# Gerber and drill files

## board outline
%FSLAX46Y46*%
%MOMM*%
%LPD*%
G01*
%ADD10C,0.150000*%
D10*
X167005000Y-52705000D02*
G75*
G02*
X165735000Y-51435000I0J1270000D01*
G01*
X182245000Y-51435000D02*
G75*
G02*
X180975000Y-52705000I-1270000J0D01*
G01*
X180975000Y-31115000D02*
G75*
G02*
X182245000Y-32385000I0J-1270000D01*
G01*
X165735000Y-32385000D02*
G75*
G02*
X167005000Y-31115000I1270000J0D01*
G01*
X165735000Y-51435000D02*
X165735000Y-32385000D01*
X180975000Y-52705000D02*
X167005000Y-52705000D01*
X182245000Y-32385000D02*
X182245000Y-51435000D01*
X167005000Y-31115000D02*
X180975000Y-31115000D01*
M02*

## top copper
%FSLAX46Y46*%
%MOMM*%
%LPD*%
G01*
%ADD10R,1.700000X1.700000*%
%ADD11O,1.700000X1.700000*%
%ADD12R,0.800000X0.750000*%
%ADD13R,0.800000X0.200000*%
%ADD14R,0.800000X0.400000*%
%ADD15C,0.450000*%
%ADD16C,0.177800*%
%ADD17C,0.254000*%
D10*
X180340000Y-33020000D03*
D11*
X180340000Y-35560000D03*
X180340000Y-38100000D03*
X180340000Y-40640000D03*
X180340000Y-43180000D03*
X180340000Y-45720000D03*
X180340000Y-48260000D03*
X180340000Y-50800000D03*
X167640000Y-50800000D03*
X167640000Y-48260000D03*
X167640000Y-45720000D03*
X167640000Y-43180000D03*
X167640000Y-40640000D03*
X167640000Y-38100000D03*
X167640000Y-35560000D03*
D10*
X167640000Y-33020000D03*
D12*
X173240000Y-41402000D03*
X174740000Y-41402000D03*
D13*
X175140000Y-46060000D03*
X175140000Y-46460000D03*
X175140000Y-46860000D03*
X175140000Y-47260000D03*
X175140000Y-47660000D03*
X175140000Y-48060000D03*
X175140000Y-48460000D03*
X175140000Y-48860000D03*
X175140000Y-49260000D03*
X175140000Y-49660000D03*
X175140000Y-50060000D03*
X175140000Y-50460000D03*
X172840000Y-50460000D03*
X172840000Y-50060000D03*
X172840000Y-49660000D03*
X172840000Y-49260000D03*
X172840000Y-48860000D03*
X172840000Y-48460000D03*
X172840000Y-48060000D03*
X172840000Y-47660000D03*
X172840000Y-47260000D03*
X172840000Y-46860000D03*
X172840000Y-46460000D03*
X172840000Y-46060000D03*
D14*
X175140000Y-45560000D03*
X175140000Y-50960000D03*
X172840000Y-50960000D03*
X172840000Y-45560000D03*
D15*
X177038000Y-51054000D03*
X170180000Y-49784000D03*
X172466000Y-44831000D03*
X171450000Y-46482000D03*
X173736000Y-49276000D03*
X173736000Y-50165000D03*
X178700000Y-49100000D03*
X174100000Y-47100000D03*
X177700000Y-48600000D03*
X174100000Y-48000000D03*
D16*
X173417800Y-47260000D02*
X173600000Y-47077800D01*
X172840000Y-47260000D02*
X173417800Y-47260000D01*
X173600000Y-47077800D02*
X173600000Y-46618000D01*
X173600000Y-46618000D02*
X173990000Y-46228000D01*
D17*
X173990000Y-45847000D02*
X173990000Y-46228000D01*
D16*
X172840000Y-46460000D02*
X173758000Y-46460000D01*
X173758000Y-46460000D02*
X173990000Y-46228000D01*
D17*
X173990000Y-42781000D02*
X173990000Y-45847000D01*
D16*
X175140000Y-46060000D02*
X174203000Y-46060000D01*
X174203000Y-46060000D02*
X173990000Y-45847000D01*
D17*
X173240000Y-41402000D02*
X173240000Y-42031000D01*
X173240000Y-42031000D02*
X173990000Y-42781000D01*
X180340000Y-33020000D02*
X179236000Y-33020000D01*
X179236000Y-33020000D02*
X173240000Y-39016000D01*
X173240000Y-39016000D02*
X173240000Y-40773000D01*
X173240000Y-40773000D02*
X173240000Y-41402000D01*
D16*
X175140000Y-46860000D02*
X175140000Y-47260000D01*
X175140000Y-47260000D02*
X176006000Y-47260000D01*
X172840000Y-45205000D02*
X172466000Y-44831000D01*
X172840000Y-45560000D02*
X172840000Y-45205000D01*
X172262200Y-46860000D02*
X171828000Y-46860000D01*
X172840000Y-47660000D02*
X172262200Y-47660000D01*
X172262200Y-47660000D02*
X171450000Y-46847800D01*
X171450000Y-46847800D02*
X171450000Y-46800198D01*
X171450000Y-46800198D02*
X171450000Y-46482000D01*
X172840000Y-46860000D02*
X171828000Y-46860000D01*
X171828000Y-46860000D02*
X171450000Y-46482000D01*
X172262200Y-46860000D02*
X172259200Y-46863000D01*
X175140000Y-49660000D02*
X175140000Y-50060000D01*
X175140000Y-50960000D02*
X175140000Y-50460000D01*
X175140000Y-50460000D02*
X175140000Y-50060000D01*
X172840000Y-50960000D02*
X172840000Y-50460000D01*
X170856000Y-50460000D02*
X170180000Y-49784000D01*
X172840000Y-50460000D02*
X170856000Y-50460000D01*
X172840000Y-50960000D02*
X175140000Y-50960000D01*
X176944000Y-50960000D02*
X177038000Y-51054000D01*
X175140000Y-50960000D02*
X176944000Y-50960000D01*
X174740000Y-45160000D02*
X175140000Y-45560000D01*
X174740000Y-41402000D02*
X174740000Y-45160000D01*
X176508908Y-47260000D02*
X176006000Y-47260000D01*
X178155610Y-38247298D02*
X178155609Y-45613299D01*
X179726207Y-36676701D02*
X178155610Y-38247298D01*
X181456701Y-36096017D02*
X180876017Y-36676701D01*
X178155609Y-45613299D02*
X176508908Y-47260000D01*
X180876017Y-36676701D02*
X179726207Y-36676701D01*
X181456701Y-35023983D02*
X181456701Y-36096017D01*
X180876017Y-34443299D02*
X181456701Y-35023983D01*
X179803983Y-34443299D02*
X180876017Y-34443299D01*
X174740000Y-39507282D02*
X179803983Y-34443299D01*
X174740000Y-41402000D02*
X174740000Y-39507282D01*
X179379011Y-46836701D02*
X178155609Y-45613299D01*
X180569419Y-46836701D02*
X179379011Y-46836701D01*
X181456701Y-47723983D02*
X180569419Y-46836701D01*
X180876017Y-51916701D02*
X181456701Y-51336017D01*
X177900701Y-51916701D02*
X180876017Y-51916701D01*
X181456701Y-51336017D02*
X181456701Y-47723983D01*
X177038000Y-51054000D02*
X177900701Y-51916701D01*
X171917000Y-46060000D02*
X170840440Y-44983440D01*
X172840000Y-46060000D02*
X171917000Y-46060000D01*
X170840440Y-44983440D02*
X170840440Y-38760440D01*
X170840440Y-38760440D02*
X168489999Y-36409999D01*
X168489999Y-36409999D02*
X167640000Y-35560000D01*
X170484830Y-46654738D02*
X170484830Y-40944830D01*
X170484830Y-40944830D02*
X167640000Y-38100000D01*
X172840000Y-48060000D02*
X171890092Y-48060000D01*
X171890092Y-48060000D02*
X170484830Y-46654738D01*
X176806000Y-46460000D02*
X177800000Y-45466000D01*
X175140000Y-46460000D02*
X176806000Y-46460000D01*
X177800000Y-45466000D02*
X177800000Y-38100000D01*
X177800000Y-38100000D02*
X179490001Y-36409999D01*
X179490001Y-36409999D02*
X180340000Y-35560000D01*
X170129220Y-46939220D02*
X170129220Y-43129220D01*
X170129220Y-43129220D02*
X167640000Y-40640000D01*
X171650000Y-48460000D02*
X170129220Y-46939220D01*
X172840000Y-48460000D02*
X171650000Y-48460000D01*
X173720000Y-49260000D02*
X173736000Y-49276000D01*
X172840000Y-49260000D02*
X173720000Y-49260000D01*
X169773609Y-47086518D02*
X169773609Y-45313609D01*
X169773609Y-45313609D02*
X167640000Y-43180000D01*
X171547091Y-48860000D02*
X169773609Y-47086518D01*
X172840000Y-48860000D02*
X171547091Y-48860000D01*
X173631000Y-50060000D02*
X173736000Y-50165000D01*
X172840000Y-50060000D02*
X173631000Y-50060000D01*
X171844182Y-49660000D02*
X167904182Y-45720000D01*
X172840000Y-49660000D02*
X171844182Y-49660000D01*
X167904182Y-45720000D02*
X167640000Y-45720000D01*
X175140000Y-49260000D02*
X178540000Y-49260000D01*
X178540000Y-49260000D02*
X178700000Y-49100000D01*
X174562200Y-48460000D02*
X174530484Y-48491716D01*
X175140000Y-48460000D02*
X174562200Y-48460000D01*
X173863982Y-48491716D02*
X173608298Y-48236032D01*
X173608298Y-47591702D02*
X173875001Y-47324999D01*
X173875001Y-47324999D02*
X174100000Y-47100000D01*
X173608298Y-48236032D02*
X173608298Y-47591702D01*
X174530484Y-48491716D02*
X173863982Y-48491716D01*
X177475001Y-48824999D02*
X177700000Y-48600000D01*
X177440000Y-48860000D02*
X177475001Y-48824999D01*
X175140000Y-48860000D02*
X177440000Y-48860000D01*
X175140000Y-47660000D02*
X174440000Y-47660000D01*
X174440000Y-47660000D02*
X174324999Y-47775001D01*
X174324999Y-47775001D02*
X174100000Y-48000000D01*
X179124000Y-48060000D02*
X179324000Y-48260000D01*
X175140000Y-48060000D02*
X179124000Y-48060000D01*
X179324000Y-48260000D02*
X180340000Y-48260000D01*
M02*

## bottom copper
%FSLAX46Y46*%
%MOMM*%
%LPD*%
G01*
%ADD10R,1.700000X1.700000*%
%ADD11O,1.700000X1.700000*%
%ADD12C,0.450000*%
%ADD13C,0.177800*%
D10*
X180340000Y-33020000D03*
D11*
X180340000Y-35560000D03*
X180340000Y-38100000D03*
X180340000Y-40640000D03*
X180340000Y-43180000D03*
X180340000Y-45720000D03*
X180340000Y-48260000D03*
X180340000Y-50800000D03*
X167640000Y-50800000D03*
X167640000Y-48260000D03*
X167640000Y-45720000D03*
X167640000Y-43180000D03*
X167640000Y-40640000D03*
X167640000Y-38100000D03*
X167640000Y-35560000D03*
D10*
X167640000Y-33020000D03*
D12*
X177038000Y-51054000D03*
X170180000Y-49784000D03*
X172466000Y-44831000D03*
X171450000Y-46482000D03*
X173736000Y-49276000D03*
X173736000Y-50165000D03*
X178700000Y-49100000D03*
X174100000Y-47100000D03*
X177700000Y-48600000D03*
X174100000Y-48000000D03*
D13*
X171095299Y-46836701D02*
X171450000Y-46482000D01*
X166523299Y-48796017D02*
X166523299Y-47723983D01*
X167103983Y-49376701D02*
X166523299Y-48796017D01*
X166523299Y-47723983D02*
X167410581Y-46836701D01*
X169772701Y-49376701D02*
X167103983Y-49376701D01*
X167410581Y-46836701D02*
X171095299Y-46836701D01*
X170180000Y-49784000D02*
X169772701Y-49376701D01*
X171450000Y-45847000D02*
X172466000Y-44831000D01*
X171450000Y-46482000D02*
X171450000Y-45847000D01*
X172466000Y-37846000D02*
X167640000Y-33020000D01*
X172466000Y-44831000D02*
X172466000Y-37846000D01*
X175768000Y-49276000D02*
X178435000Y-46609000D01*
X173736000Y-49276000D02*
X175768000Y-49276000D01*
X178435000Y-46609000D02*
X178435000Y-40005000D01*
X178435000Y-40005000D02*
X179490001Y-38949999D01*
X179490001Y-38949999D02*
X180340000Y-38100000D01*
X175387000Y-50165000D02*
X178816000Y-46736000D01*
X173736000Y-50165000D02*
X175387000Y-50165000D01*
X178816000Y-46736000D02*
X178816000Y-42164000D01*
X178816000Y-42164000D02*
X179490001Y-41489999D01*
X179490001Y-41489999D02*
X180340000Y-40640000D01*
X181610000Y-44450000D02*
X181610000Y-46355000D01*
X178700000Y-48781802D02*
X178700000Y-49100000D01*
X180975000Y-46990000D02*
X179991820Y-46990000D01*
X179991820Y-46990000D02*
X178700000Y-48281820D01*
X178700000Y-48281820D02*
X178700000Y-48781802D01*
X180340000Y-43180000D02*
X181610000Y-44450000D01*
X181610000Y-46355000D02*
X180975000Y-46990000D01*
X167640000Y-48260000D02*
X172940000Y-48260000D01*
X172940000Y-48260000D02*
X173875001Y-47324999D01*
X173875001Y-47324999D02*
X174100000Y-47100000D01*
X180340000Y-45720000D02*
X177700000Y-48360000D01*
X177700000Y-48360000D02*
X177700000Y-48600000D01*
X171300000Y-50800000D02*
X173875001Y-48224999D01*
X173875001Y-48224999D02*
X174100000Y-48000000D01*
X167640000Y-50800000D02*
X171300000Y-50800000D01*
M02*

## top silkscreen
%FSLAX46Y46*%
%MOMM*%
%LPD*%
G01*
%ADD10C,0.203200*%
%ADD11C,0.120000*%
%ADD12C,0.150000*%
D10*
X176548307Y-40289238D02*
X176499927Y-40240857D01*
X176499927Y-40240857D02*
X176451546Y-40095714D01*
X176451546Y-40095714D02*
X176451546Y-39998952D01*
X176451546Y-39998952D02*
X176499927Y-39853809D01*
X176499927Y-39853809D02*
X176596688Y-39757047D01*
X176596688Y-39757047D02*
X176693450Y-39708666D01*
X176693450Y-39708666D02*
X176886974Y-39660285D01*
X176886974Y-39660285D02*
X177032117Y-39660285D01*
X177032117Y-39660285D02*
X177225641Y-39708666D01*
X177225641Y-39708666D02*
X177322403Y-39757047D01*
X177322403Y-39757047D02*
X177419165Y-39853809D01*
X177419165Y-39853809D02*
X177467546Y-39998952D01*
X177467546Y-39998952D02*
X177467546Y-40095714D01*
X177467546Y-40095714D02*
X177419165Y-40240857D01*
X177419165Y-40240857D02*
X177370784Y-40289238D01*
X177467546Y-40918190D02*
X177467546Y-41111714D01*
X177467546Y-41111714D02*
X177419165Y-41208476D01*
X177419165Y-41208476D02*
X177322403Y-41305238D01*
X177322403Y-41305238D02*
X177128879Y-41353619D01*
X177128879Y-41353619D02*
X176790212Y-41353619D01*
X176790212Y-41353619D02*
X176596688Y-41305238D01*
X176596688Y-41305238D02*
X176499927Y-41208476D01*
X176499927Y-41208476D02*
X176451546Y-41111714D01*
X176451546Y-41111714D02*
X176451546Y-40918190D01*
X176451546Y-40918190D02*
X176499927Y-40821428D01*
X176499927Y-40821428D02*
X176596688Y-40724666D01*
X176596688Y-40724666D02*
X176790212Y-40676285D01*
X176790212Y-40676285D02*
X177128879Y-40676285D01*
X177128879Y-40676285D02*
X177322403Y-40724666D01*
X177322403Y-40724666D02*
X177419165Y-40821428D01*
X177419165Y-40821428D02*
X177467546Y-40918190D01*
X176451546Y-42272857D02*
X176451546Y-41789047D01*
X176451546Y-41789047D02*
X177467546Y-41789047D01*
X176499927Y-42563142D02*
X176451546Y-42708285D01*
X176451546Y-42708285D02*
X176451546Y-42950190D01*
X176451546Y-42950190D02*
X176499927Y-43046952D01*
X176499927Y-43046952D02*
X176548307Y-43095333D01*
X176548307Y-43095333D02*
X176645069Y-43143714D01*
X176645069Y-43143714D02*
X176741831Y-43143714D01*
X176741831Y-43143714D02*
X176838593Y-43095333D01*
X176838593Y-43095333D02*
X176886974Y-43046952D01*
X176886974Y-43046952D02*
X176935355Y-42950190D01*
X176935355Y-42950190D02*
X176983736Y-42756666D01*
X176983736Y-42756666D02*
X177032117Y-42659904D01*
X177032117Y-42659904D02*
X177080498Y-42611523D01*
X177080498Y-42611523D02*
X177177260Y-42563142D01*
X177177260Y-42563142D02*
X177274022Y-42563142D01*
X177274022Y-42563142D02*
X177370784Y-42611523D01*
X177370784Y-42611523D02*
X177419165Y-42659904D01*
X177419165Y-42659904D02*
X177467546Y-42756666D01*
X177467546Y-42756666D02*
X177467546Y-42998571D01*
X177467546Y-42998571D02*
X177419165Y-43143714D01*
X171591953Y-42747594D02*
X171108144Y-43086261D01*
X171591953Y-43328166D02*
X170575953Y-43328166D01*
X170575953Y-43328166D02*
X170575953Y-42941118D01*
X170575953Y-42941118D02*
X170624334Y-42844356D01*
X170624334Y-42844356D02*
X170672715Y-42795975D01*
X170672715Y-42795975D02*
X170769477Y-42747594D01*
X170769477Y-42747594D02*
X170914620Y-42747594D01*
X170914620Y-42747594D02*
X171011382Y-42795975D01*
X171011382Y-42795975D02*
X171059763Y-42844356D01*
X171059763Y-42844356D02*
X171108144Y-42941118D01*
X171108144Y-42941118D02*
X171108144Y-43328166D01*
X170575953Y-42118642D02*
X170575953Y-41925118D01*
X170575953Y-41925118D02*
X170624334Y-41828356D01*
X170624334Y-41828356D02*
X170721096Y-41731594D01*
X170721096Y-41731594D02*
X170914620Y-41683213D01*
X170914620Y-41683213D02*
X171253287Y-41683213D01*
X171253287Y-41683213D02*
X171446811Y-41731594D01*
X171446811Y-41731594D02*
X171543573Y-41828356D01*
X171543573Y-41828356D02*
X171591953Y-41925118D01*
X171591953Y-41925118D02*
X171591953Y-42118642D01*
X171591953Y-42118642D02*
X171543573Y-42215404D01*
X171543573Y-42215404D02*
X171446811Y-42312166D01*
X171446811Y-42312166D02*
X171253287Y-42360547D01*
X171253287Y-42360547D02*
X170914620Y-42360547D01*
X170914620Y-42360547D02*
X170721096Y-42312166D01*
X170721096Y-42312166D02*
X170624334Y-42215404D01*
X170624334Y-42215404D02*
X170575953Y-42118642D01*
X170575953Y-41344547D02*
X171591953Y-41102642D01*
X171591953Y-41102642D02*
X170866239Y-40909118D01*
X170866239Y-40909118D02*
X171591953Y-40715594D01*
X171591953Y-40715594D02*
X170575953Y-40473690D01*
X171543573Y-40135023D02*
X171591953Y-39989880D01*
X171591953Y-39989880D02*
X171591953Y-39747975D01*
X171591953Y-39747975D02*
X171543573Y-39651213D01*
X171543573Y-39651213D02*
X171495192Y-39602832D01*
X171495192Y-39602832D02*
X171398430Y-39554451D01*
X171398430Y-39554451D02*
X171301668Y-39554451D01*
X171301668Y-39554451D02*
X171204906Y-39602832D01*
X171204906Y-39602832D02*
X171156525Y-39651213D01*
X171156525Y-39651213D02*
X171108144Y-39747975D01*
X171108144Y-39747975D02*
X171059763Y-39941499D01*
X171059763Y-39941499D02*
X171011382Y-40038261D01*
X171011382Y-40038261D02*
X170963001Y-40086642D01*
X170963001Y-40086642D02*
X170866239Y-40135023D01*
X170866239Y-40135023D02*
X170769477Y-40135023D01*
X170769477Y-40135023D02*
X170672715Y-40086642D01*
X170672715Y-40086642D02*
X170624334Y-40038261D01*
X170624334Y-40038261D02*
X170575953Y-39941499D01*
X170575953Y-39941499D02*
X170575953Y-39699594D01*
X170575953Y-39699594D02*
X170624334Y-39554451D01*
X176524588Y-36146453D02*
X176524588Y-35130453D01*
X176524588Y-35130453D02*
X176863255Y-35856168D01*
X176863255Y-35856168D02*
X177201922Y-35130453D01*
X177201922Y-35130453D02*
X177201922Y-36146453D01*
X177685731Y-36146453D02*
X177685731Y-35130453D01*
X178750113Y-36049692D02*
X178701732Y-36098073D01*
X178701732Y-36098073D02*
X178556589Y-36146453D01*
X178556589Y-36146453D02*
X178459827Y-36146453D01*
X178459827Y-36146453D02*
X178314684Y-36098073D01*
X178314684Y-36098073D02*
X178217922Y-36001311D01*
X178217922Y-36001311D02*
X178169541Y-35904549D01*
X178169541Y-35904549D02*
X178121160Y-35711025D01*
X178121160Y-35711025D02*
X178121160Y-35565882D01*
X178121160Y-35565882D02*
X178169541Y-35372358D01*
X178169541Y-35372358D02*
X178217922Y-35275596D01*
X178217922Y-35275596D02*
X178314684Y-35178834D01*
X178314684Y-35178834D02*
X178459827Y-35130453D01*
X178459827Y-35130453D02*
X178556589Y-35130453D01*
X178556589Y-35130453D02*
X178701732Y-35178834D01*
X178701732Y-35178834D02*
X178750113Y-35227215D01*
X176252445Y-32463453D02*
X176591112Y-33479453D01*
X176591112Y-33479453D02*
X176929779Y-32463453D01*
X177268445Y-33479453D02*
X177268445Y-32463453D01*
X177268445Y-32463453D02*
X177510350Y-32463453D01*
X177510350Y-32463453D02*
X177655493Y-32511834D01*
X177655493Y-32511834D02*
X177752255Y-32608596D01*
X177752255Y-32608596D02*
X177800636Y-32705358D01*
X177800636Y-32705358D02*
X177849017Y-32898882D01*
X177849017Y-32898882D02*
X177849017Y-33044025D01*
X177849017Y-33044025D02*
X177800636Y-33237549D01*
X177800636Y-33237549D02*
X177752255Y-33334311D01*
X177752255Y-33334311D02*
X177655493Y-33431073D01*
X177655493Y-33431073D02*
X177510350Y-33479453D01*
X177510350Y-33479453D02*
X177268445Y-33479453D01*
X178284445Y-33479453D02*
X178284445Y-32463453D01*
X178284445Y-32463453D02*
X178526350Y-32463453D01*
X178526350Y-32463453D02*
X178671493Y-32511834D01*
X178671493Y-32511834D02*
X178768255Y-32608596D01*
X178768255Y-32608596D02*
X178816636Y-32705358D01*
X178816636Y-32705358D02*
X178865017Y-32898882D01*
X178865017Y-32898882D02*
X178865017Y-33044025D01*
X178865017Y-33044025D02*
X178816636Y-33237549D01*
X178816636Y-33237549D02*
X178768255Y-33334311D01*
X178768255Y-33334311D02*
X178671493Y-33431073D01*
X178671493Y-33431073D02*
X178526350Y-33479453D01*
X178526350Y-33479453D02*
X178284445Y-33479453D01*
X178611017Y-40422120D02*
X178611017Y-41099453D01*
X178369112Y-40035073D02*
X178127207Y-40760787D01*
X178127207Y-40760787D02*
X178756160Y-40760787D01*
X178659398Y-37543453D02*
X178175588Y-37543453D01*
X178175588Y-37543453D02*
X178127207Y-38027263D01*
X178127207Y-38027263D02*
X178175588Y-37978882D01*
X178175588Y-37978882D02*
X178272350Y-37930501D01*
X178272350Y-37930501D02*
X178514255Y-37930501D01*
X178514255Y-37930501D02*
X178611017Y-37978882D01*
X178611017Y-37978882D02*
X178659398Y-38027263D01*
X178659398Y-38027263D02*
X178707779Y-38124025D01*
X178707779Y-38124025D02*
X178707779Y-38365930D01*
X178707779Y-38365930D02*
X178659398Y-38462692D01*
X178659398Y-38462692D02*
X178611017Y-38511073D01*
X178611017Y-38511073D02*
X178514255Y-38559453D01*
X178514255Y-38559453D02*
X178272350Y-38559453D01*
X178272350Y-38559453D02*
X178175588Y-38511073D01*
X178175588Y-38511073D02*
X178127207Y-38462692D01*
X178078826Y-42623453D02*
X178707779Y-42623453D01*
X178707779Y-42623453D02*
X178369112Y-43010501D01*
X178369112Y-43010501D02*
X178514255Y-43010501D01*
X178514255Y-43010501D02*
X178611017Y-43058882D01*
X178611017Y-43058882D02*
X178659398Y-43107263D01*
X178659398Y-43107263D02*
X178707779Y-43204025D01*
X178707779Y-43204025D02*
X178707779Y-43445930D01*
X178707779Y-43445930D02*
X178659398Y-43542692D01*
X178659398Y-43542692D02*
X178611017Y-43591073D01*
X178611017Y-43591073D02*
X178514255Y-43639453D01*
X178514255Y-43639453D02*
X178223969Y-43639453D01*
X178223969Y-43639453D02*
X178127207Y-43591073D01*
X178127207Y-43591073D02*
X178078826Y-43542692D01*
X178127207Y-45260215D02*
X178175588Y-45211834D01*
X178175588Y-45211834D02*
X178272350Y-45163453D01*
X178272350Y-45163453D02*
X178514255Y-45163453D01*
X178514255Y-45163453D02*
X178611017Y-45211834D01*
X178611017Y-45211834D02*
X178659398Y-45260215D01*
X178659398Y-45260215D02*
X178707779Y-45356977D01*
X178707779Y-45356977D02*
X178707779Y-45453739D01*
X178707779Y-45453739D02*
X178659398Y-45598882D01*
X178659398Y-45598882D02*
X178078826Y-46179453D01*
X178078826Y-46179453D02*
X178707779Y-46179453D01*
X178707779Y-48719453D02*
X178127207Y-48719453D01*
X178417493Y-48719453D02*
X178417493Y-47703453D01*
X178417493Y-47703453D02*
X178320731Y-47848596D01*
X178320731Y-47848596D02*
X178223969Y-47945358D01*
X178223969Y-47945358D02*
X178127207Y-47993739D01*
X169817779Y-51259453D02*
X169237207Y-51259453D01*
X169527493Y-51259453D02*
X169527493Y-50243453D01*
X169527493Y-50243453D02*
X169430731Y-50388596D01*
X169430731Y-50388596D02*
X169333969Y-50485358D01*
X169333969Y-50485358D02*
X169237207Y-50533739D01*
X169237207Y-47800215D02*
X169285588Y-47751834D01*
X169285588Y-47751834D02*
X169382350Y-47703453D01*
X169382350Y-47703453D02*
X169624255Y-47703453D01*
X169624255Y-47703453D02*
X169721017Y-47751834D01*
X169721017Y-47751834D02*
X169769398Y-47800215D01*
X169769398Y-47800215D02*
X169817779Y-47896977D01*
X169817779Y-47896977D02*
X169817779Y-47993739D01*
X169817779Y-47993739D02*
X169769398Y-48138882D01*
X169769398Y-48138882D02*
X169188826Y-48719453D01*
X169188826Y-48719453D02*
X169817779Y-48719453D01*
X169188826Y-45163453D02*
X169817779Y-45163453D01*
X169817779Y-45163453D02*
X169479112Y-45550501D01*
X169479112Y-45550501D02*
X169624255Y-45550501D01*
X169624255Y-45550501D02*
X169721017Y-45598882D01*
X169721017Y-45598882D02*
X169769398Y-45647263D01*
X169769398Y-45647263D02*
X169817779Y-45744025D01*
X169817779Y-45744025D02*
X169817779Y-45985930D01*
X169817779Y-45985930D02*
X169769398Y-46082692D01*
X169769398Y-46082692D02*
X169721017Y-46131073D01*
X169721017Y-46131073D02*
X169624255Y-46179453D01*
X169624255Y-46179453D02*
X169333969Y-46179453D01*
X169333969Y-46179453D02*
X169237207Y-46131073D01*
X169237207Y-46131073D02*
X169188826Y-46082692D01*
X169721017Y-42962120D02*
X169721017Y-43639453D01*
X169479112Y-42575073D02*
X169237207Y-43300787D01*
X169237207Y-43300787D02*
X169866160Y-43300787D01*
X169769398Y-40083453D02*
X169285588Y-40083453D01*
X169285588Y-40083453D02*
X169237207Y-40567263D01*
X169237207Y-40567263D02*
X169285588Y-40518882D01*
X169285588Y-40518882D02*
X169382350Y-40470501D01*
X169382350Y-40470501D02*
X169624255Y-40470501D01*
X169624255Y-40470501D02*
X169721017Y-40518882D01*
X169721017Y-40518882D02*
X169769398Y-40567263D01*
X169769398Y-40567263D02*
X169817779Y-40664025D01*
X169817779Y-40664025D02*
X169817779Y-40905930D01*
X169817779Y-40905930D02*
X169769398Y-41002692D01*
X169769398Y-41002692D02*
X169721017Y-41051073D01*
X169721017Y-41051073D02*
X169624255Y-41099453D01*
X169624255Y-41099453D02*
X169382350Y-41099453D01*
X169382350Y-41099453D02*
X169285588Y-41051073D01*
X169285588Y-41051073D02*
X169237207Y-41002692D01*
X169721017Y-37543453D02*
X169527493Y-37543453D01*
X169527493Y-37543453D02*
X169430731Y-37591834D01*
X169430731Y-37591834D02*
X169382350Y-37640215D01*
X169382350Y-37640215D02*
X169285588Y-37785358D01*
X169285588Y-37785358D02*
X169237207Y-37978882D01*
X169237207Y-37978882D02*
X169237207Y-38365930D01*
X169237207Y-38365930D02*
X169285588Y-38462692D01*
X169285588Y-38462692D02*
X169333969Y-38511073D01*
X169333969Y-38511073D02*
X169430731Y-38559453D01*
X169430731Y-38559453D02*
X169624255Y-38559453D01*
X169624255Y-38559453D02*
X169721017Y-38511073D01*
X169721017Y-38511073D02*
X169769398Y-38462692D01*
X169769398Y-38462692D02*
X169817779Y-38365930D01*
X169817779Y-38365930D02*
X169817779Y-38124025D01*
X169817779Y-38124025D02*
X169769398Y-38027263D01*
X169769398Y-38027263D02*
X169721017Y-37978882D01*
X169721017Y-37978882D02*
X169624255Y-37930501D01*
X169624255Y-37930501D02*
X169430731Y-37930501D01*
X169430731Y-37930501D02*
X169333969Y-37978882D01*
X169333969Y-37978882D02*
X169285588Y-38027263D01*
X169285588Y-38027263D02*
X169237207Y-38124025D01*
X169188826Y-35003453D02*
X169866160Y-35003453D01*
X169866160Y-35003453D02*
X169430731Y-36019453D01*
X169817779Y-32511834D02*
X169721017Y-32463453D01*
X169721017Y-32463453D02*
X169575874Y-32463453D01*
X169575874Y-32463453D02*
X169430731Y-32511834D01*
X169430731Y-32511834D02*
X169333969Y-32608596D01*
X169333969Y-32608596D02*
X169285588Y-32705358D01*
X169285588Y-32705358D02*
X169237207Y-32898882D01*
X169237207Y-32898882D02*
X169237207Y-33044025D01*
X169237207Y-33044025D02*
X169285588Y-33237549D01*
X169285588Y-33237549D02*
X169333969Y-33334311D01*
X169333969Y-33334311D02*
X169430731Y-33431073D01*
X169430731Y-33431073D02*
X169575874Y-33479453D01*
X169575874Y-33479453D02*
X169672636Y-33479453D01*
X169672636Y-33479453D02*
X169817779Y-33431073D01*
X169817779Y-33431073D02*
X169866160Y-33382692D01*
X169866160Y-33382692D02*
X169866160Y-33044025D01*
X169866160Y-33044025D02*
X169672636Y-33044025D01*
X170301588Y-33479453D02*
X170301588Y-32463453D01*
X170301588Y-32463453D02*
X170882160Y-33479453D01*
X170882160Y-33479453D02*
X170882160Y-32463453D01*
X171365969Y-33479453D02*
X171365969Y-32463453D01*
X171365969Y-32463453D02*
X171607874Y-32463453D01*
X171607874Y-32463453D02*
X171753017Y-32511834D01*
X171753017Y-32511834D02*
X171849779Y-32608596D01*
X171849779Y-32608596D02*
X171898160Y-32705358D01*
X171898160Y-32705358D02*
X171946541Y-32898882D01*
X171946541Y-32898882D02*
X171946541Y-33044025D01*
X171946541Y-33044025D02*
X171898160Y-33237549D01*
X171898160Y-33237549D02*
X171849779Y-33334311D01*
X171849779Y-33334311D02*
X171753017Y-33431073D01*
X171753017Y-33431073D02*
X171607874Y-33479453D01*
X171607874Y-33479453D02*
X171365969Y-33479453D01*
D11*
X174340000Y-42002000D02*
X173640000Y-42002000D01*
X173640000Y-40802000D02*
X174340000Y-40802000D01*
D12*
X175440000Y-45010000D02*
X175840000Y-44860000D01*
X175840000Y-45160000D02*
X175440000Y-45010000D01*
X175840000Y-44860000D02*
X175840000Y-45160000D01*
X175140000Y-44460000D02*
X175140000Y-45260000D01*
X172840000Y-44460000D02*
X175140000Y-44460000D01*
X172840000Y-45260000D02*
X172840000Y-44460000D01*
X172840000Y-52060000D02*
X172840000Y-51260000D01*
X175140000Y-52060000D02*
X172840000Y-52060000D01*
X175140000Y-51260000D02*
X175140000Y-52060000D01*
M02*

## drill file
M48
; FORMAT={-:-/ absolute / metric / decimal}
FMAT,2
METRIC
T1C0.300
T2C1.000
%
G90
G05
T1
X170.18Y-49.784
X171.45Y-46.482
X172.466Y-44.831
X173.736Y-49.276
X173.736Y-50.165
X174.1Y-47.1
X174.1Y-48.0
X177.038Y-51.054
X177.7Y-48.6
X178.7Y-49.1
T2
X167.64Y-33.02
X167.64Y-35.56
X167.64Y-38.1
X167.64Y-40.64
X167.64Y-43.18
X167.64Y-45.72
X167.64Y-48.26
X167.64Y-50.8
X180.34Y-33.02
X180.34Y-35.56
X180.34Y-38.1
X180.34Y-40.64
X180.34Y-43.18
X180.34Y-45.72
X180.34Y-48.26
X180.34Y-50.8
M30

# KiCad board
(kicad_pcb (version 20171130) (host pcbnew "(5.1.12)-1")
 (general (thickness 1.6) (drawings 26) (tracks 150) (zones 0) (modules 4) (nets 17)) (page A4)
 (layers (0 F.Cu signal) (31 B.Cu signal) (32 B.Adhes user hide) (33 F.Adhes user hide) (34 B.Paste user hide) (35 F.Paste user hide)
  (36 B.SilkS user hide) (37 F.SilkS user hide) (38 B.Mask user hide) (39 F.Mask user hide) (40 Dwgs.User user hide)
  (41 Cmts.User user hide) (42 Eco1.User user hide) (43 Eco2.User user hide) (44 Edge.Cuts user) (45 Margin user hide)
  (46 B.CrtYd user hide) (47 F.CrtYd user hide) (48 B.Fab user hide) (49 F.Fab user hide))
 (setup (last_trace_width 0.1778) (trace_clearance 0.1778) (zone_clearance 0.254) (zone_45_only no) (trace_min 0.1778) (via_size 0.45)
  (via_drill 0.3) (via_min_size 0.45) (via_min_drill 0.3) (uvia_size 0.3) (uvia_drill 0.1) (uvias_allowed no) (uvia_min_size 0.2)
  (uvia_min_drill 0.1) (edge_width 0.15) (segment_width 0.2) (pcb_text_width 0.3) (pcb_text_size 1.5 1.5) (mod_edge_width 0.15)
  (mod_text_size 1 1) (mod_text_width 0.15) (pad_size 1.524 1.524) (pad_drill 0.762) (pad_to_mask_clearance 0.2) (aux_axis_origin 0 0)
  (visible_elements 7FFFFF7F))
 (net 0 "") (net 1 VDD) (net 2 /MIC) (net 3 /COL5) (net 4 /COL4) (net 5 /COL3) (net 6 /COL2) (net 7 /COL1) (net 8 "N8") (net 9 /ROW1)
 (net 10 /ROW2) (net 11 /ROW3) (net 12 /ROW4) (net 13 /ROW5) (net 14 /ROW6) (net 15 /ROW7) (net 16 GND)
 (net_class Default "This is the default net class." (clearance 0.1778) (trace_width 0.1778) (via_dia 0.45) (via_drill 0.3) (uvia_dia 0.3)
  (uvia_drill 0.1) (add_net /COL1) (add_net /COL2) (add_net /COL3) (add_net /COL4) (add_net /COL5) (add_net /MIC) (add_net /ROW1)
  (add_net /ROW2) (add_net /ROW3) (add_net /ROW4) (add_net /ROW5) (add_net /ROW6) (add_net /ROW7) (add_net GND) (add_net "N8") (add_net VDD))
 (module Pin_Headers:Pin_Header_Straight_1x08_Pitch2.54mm (layer B.Cu) (at 180.34 33.02 180)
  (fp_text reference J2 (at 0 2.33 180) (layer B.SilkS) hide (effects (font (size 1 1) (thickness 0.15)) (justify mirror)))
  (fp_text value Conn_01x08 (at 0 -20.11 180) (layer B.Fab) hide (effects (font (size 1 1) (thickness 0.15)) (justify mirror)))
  (pad 1 thru_hole rect (at 0 0 180) (size 1.7 1.7) (drill 1) (layers *.Cu *.Mask) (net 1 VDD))
  (pad 2 thru_hole oval (at 0 -2.54 180) (size 1.7 1.7) (drill 1) (layers *.Cu *.Mask) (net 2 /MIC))
  (pad 3 thru_hole oval (at 0 -5.08 180) (size 1.7 1.7) (drill 1) (layers *.Cu *.Mask) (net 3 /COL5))
  (pad 4 thru_hole oval (at 0 -7.62 180) (size 1.7 1.7) (drill 1) (layers *.Cu *.Mask) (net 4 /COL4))
  (pad 5 thru_hole oval (at 0 -10.16 180) (size 1.7 1.7) (drill 1) (layers *.Cu *.Mask) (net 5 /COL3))
  (pad 6 thru_hole oval (at 0 -12.7 180) (size 1.7 1.7) (drill 1) (layers *.Cu *.Mask) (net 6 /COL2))
  (pad 7 thru_hole oval (at 0 -15.24 180) (size 1.7 1.7) (drill 1) (layers *.Cu *.Mask) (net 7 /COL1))
  (pad 8 thru_hole oval (at 0 -17.78 180) (size 1.7 1.7) (drill 1) (layers *.Cu *.Mask) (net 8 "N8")))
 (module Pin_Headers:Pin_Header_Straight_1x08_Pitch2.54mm (layer B.Cu) (at 167.64 33.02 180)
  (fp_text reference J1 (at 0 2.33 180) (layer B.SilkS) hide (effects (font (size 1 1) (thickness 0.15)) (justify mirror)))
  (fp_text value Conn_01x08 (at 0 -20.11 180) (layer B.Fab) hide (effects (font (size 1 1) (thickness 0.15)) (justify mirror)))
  (pad 8 thru_hole oval (at 0 -17.78 180) (size 1.7 1.7) (drill 1) (layers *.Cu *.Mask) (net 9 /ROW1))
  (pad 7 thru_hole oval (at 0 -15.24 180) (size 1.7 1.7) (drill 1) (layers *.Cu *.Mask) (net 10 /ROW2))
  (pad 6 thru_hole oval (at 0 -12.7 180) (size 1.7 1.7) (drill 1) (layers *.Cu *.Mask) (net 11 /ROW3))
  (pad 5 thru_hole oval (at 0 -10.16 180) (size 1.7 1.7) (drill 1) (layers *.Cu *.Mask) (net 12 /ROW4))
  (pad 4 thru_hole oval (at 0 -7.62 180) (size 1.7 1.7) (drill 1) (layers *.Cu *.Mask) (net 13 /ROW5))
  (pad 3 thru_hole oval (at 0 -5.08 180) (size 1.7 1.7) (drill 1) (layers *.Cu *.Mask) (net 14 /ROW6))
  (pad 2 thru_hole oval (at 0 -2.54 180) (size 1.7 1.7) (drill 1) (layers *.Cu *.Mask) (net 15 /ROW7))
  (pad 1 thru_hole rect (at 0 0 180) (size 1.7 1.7) (drill 1) (layers *.Cu *.Mask) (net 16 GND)))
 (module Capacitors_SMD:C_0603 (layer F.Cu) (at 173.99 41.402)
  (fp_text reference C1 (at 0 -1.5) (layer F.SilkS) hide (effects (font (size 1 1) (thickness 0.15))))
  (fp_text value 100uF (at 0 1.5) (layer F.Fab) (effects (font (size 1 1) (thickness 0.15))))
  (fp_line (start 0.35 0.6) (end -0.35 0.6) (layer F.SilkS) (width 0.12))
  (fp_line (start -0.35 -0.6) (end 0.35 -0.6) (layer F.SilkS) (width 0.12))
  (pad 1 smd rect (at -0.75 0) (size 0.8 0.75) (layers F.Cu F.Paste F.Mask) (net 1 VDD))
  (pad 2 smd rect (at 0.75 0) (size 0.8 0.75) (layers F.Cu F.Paste F.Mask) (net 16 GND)))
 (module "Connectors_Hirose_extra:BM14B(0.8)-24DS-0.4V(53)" (layer F.Cu) (at 173.99 48.26 270)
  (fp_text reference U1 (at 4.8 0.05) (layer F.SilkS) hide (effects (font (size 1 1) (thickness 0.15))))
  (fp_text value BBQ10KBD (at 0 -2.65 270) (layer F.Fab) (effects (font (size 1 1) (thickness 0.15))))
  (fp_line (start -3.25 -1.45) (end -3.4 -1.85) (layer F.SilkS) (width 0.15))
  (fp_line (start -3.1 -1.85) (end -3.25 -1.45) (layer F.SilkS) (width 0.15))
  (fp_line (start -3.4 -1.85) (end -3.1 -1.85) (layer F.SilkS) (width 0.15))
  (fp_line (start -3.8 -1.15) (end -3 -1.15) (layer F.SilkS) (width 0.15))
  (fp_line (start -3.8 1.15) (end -3.8 -1.15) (layer F.SilkS) (width 0.15))
  (fp_line (start -3 1.15) (end -3.8 1.15) (layer F.SilkS) (width 0.15))
  (fp_line (start 3.8 1.15) (end 3 1.15) (layer F.SilkS) (width 0.15))
  (fp_line (start 3.8 -1.15) (end 3.8 1.15) (layer F.SilkS) (width 0.15))
  (fp_line (start 3 -1.15) (end 3.8 -1.15) (layer F.SilkS) (width 0.15))
  (pad 2 smd rect (at -2.2 -1.15 270) (size 0.2 0.8) (layers F.Cu F.Paste F.Mask) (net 1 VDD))
  (pad 3 smd rect (at -1.8 -1.15 270) (size 0.2 0.8) (layers F.Cu F.Paste F.Mask) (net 2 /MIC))
  (pad 4 smd rect (at -1.4 -1.15 270) (size 0.2 0.8) (layers F.Cu F.Paste F.Mask) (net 16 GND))
  (pad 5 smd rect (at -1 -1.15 270) (size 0.2 0.8) (layers F.Cu F.Paste F.Mask) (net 16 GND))
  (pad 6 smd rect (at -0.6 -1.15 270) (size 0.2 0.8) (layers F.Cu F.Paste F.Mask) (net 9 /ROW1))
  (pad 7 smd rect (at -0.2 -1.15 270) (size 0.2 0.8) (layers F.Cu F.Paste F.Mask) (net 7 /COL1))
  (pad 8 smd rect (at 0.2 -1.15 270) (size 0.2 0.8) (layers F.Cu F.Paste F.Mask) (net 10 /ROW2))
  (pad 9 smd rect (at 0.6 -1.15 270) (size 0.2 0.8) (layers F.Cu F.Paste F.Mask) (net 6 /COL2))
  (pad 10 smd rect (at 1 -1.15 270) (size 0.2 0.8) (layers F.Cu F.Paste F.Mask) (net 5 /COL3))
  (pad 11 smd rect (at 1.4 -1.15 270) (size 0.2 0.8) (layers F.Cu F.Paste F.Mask) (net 16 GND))
  (pad 12 smd rect (at 1.8 -1.15 270) (size 0.2 0.8) (layers F.Cu F.Paste F.Mask) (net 16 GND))
  (pad 13 smd rect (at 2.2 -1.15 270) (size 0.2 0.8) (layers F.Cu F.Paste F.Mask) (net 16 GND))
  (pad 16 smd rect (at 2.2 1.15 270) (size 0.2 0.8) (layers F.Cu F.Paste F.Mask) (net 16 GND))
  (pad 17 smd rect (at 1.8 1.15 270) (size 0.2 0.8) (layers F.Cu F.Paste F.Mask) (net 4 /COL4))
  (pad 18 smd rect (at 1.4 1.15 270) (size 0.2 0.8) (layers F.Cu F.Paste F.Mask) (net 11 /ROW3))
  (pad 19 smd rect (at 1 1.15 270) (size 0.2 0.8) (layers F.Cu F.Paste F.Mask) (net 3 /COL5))
  (pad 20 smd rect (at 0.6 1.15 270) (size 0.2 0.8) (layers F.Cu F.Paste F.Mask) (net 12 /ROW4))
  (pad 21 smd rect (at 0.2 1.15 270) (size 0.2 0.8) (layers F.Cu F.Paste F.Mask) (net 13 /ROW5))
  (pad 22 smd rect (at -0.2 1.15 270) (size 0.2 0.8) (layers F.Cu F.Paste F.Mask) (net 14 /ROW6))
  (pad 23 smd rect (at -0.6 1.15 270) (size 0.2 0.8) (layers F.Cu F.Paste F.Mask) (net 16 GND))
  (pad 24 smd rect (at -1 1.15 270) (size 0.2 0.8) (layers F.Cu F.Paste F.Mask) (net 1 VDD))
  (pad 25 smd rect (at -1.4 1.15 270) (size 0.2 0.8) (layers F.Cu F.Paste F.Mask) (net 16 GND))
  (pad 26 smd rect (at -1.8 1.15 270) (size 0.2 0.8) (layers F.Cu F.Paste F.Mask) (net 1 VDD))
  (pad 27 smd rect (at -2.2 1.15 270) (size 0.2 0.8) (layers F.Cu F.Paste F.Mask) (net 15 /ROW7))
  (pad 1 smd rect (at -2.7 -1.15 270) (size 0.4 0.8) (layers F.Cu F.Paste F.Mask) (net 16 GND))
  (pad 14 smd rect (at 2.7 -1.15 270) (size 0.4 0.8) (layers F.Cu F.Paste F.Mask) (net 16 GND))
  (pad 15 smd rect (at 2.7 1.15 270) (size 0.4 0.8) (layers F.Cu F.Paste F.Mask) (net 16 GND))
  (pad 28 smd rect (at -2.7 1.15 270) (size 0.4 0.8) (layers F.Cu F.Paste F.Mask) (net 16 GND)))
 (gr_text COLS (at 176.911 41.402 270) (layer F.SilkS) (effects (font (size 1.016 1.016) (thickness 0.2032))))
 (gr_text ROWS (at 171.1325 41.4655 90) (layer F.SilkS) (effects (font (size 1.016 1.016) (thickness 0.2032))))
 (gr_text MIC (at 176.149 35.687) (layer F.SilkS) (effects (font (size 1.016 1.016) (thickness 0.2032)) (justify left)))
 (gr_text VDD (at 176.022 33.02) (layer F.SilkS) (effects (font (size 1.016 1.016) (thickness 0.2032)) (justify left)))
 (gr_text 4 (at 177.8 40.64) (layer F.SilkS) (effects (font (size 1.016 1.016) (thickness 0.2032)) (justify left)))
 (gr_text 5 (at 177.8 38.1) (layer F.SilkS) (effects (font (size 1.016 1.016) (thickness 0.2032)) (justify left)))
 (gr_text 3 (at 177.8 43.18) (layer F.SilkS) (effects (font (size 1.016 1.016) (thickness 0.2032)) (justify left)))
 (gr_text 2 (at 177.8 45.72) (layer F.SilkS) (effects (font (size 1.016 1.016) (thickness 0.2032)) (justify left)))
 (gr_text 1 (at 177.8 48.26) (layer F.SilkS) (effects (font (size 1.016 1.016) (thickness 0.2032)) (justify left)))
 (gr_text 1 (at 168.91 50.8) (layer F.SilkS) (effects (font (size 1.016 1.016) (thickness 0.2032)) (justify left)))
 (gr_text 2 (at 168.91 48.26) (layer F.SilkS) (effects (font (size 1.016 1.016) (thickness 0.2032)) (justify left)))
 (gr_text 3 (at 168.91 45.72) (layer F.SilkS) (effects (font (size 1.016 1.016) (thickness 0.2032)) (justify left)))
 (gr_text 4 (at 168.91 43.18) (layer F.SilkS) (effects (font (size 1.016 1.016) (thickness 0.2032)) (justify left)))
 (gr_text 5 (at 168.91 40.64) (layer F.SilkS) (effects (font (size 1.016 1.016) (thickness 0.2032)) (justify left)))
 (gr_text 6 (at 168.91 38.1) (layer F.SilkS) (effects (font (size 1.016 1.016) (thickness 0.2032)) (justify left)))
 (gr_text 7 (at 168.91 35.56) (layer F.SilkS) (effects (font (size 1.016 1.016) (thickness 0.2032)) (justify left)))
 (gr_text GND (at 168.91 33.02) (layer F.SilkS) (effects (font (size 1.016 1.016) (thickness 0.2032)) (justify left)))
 (gr_arc (start 167.005 51.435) (end 165.735 51.435) (angle -90) (layer Edge.Cuts) (width 0.15))
 (gr_arc (start 180.975 51.435) (end 180.975 52.705) (angle -90) (layer Edge.Cuts) (width 0.15))
 (gr_arc (start 180.975 32.385) (end 182.245 32.385) (angle -90) (layer Edge.Cuts) (width 0.15))
 (gr_arc (start 167.005 32.385) (end 167.005 31.115) (angle -90) (layer Edge.Cuts) (width 0.15))
 (gr_line (start 165.735 51.435) (end 165.735 32.385) (layer Edge.Cuts) (width 0.15))
 (gr_line (start 180.975 52.705) (end 167.005 52.705) (layer Edge.Cuts) (width 0.15))
 (gr_line (start 182.245 32.385) (end 182.245 51.435) (layer Edge.Cuts) (width 0.15))
 (gr_line (start 167.005 31.115) (end 180.975 31.115) (layer Edge.Cuts) (width 0.15))
 (segment (start 173.4178 47.26) (end 173.6 47.0778) (width 0.1778) (layer F.Cu) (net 1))
 (segment (start 172.84 47.26) (end 173.4178 47.26) (width 0.1778) (layer F.Cu) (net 1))
 (segment (start 173.6 47.0778) (end 173.6 46.618) (width 0.1778) (layer F.Cu) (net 1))
 (segment (start 173.6 46.618) (end 173.99 46.228) (width 0.1778) (layer F.Cu) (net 1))
 (segment (start 173.99 45.847) (end 173.99 46.228) (width 0.254) (layer F.Cu) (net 1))
 (segment (start 172.84 46.46) (end 173.758 46.46) (width 0.1778) (layer F.Cu) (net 1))
 (segment (start 173.758 46.46) (end 173.99 46.228) (width 0.1778) (layer F.Cu) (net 1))
 (segment (start 173.99 42.781) (end 173.99 45.847) (width 0.254) (layer F.Cu) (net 1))
 (segment (start 175.14 46.06) (end 174.203 46.06) (width 0.1778) (layer F.Cu) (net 1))
 (segment (start 174.203 46.06) (end 173.99 45.847) (width 0.1778) (layer F.Cu) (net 1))
 (segment (start 173.24 41.402) (end 173.24 42.031) (width 0.254) (layer F.Cu) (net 1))
 (segment (start 173.24 42.031) (end 173.99 42.781) (width 0.254) (layer F.Cu) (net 1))
 (segment (start 180.34 33.02) (end 179.236 33.02) (width 0.254) (layer F.Cu) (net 1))
 (segment (start 179.236 33.02) (end 173.24 39.016) (width 0.254) (layer F.Cu) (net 1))
 (segment (start 173.24 39.016) (end 173.24 40.773) (width 0.254) (layer F.Cu) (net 1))
 (segment (start 173.24 40.773) (end 173.24 41.402) (width 0.254) (layer F.Cu) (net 1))
 (via (at 177.038 51.054) (size 0.45) (drill 0.3) (layers F.Cu B.Cu) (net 16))
 (via (at 170.18 49.784) (size 0.45) (drill 0.3) (layers F.Cu B.Cu) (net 16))
 (segment (start 175.14 46.86) (end 175.14 47.26) (width 0.1778) (layer F.Cu) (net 16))
 (segment (start 175.14 47.26) (end 176.006 47.26) (width 0.1778) (layer F.Cu) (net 16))
 (segment (start 172.84 45.205) (end 172.466 44.831) (width 0.1778) (layer F.Cu) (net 16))
 (segment (start 172.84 45.56) (end 172.84 45.205) (width 0.1778) (layer F.Cu) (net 16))
 (via (at 172.466 44.831) (size 0.45) (drill 0.3) (layers F.Cu B.Cu) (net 16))
 (segment (start 172.2622 46.86) (end 171.828 46.86) (width 0.1778) (layer F.Cu) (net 16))
 (segment (start 172.84 47.66) (end 172.2622 47.66) (width 0.1778) (layer F.Cu) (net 16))
 (segment (start 172.2622 47.66) (end 171.45 46.8478) (width 0.1778) (layer F.Cu) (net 16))
 (segment (start 171.45 46.8478) (end 171.45 46.800198) (width 0.1778) (layer F.Cu) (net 16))
 (segment (start 171.45 46.800198) (end 171.45 46.482) (width 0.1778) (layer F.Cu) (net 16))
 (segment (start 172.84 46.86) (end 171.828 46.86) (width 0.1778) (layer F.Cu) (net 16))
 (segment (start 171.828 46.86) (end 171.45 46.482) (width 0.1778) (layer F.Cu) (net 16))
 (via (at 171.45 46.482) (size 0.45) (drill 0.3) (layers F.Cu B.Cu) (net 16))
 (segment (start 172.2622 46.86) (end 172.2592 46.863) (width 0.1778) (layer F.Cu) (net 16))
 (segment (start 175.14 49.66) (end 175.14 50.06) (width 0.1778) (layer F.Cu) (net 16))
 (segment (start 175.14 50.96) (end 175.14 50.46) (width 0.1778) (layer F.Cu) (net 16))
 (segment (start 175.14 50.46) (end 175.14 50.06) (width 0.1778) (layer F.Cu) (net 16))
 (segment (start 172.84 50.96) (end 172.84 50.46) (width 0.1778) (layer F.Cu) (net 16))
 (segment (start 170.856 50.46) (end 170.18 49.784) (width 0.1778) (layer F.Cu) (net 16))
 (segment (start 172.84 50.46) (end 170.856 50.46) (width 0.1778) (layer F.Cu) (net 16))
 (segment (start 172.84 50.96) (end 175.14 50.96) (width 0.1778) (layer F.Cu) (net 16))
 (segment (start 176.944 50.96) (end 177.038 51.054) (width 0.1778) (layer F.Cu) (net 16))
 (segment (start 175.14 50.96) (end 176.944 50.96) (width 0.1778) (layer F.Cu) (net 16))
 (segment (start 171.095299 46.836701) (end 171.45 46.482) (width 0.1778) (layer B.Cu) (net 16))
 (segment (start 166.523299 48.796017) (end 166.523299 47.723983) (width 0.1778) (layer B.Cu) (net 16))
 (segment (start 167.103983 49.376701) (end 166.523299 48.796017) (width 0.1778) (layer B.Cu) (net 16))
 (segment (start 166.523299 47.723983) (end 167.410581 46.836701) (width 0.1778) (layer B.Cu) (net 16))
 (segment (start 169.772701 49.376701) (end 167.103983 49.376701) (width 0.1778) (layer B.Cu) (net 16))
 (segment (start 167.410581 46.836701) (end 171.095299 46.836701) (width 0.1778) (layer B.Cu) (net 16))
 (segment (start 170.18 49.784) (end 169.772701 49.376701) (width 0.1778) (layer B.Cu) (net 16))
 (segment (start 171.45 45.847) (end 172.466 44.831) (width 0.1778) (layer B.Cu) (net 16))
 (segment (start 171.45 46.482) (end 171.45 45.847) (width 0.1778) (layer B.Cu) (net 16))
 (segment (start 172.466 37.846) (end 167.64 33.02) (width 0.1778) (layer B.Cu) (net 16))
 (segment (start 172.466 44.831) (end 172.466 37.846) (width 0.1778) (layer B.Cu) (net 16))
 (segment (start 174.74 45.16) (end 175.14 45.56) (width 0.1778) (layer F.Cu) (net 16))
 (segment (start 174.74 41.402) (end 174.74 45.16) (width 0.1778) (layer F.Cu) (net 16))
 (segment (start 176.508908 47.26) (end 176.006 47.26) (width 0.1778) (layer F.Cu) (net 16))
 (segment (start 178.15561 38.247298) (end 178.155609 45.613299) (width 0.1778) (layer F.Cu) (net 16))
 (segment (start 179.726207 36.676701) (end 178.15561 38.247298) (width 0.1778) (layer F.Cu) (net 16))
 (segment (start 181.456701 36.096017) (end 180.876017 36.676701) (width 0.1778) (layer F.Cu) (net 16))
 (segment (start 178.155609 45.613299) (end 176.508908 47.26) (width 0.1778) (layer F.Cu) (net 16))
 (segment (start 180.876017 36.676701) (end 179.726207 36.676701) (width 0.1778) (layer F.Cu) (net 16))
 (segment (start 181.456701 35.023983) (end 181.456701 36.096017) (width 0.1778) (layer F.Cu) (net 16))
 (segment (start 180.876017 34.443299) (end 181.456701 35.023983) (width 0.1778) (layer F.Cu) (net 16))
 (segment (start 179.803983 34.443299) (end 180.876017 34.443299) (width 0.1778) (layer F.Cu) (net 16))
 (segment (start 174.74 39.507282) (end 179.803983 34.443299) (width 0.1778) (layer F.Cu) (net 16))
 (segment (start 174.74 41.402) (end 174.74 39.507282) (width 0.1778) (layer F.Cu) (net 16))
 (segment (start 179.379011 46.836701) (end 178.155609 45.613299) (width 0.1778) (layer F.Cu) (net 16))
 (segment (start 180.569419 46.836701) (end 179.379011 46.836701) (width 0.1778) (layer F.Cu) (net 16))
 (segment (start 181.456701 47.723983) (end 180.569419 46.836701) (width 0.1778) (layer F.Cu) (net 16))
 (segment (start 180.876017 51.916701) (end 181.456701 51.336017) (width 0.1778) (layer F.Cu) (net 16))
 (segment (start 177.900701 51.916701) (end 180.876017 51.916701) (width 0.1778) (layer F.Cu) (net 16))
 (segment (start 181.456701 51.336017) (end 181.456701 47.723983) (width 0.1778) (layer F.Cu) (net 16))
 (segment (start 177.038 51.054) (end 177.900701 51.916701) (width 0.1778) (layer F.Cu) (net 16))
 (segment (start 171.917 46.06) (end 170.84044 44.98344) (width 0.1778) (layer F.Cu) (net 15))
 (segment (start 172.84 46.06) (end 171.917 46.06) (width 0.1778) (layer F.Cu) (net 15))
 (segment (start 170.84044 44.98344) (end 170.84044 38.76044) (width 0.1778) (layer F.Cu) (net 15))
 (segment (start 170.84044 38.76044) (end 168.489999 36.409999) (width 0.1778) (layer F.Cu) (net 15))
 (segment (start 168.489999 36.409999) (end 167.64 35.56) (width 0.1778) (layer F.Cu) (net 15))
 (segment (start 170.48483 46.654738) (end 170.48483 40.94483) (width 0.1778) (layer F.Cu) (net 14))
 (segment (start 170.48483 40.94483) (end 167.64 38.1) (width 0.1778) (layer F.Cu) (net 14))
 (segment (start 172.84 48.06) (end 171.890092 48.06) (width 0.1778) (layer F.Cu) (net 14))
 (segment (start 171.890092 48.06) (end 170.48483 46.654738) (width 0.1778) (layer F.Cu) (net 14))
 (segment (start 176.806 46.46) (end 177.8 45.466) (width 0.1778) (layer F.Cu) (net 2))
 (segment (start 175.14 46.46) (end 176.806 46.46) (width 0.1778) (layer F.Cu) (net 2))
 (segment (start 177.8 45.466) (end 177.8 38.1) (width 0.1778) (layer F.Cu) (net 2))
 (segment (start 177.8 38.1) (end 179.490001 36.409999) (width 0.1778) (layer F.Cu) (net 2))
 (segment (start 179.490001 36.409999) (end 180.34 35.56) (width 0.1778) (layer F.Cu) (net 2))
 (segment (start 170.12922 46.93922) (end 170.12922 43.12922) (width 0.1778) (layer F.Cu) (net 13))
 (segment (start 170.12922 43.12922) (end 167.64 40.64) (width 0.1778) (layer F.Cu) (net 13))
 (segment (start 171.65 48.46) (end 170.12922 46.93922) (width 0.1778) (layer F.Cu) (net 13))
 (segment (start 172.84 48.46) (end 171.65 48.46) (width 0.1778) (layer F.Cu) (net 13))
 (segment (start 175.768 49.276) (end 178.435 46.609) (width 0.1778) (layer B.Cu) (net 3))
 (segment (start 173.736 49.276) (end 175.768 49.276) (width 0.1778) (layer B.Cu) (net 3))
 (segment (start 178.435 46.609) (end 178.435 40.005) (width 0.1778) (layer B.Cu) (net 3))
 (segment (start 178.435 40.005) (end 179.490001 38.949999) (width 0.1778) (layer B.Cu) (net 3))
 (segment (start 179.490001 38.949999) (end 180.34 38.1) (width 0.1778) (layer B.Cu) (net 3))
 (segment (start 173.72 49.26) (end 173.736 49.276) (width 0.1778) (layer F.Cu) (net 3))
 (segment (start 172.84 49.26) (end 173.72 49.26) (width 0.1778) (layer F.Cu) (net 3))
 (via (at 173.736 49.276) (size 0.45) (drill 0.3) (layers F.Cu B.Cu) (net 3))
 (segment (start 169.773609 47.086518) (end 169.773609 45.313609) (width 0.1778) (layer F.Cu) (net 12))
 (segment (start 169.773609 45.313609) (end 167.64 43.18) (width 0.1778) (layer F.Cu) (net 12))
 (segment (start 171.547091 48.86) (end 169.773609 47.086518) (width 0.1778) (layer F.Cu) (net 12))
 (segment (start 172.84 48.86) (end 171.547091 48.86) (width 0.1778) (layer F.Cu) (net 12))
 (segment (start 175.387 50.165) (end 178.816 46.736) (width 0.1778) (layer B.Cu) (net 4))
 (segment (start 173.736 50.165) (end 175.387 50.165) (width 0.1778) (layer B.Cu) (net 4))
 (segment (start 178.816 46.736) (end 178.816 42.164) (width 0.1778) (layer B.Cu) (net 4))
 (segment (start 178.816 42.164) (end 179.490001 41.489999) (width 0.1778) (layer B.Cu) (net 4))
 (segment (start 179.490001 41.489999) (end 180.34 40.64) (width 0.1778) (layer B.Cu) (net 4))
 (segment (start 173.631 50.06) (end 173.736 50.165) (width 0.1778) (layer F.Cu) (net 4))
 (segment (start 172.84 50.06) (end 173.631 50.06) (width 0.1778) (layer F.Cu) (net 4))
 (via (at 173.736 50.165) (size 0.45) (drill 0.3) (layers F.Cu B.Cu) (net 4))
 (segment (start 171.844182 49.66) (end 167.904182 45.72) (width 0.1778) (layer F.Cu) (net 11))
 (segment (start 172.84 49.66) (end 171.844182 49.66) (width 0.1778) (layer F.Cu) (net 11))
 (segment (start 167.904182 45.72) (end 167.64 45.72) (width 0.1778) (layer F.Cu) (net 11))
 (segment (start 181.61 44.45) (end 181.61 46.355) (width 0.1778) (layer B.Cu) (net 5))
 (segment (start 178.7 48.781802) (end 178.7 49.1) (width 0.1778) (layer B.Cu) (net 5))
 (segment (start 180.975 46.99) (end 179.99182 46.99) (width 0.1778) (layer B.Cu) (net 5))
 (segment (start 175.14 49.26) (end 178.54 49.26) (width 0.1778) (layer F.Cu) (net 5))
 (segment (start 178.54 49.26) (end 178.7 49.1) (width 0.1778) (layer F.Cu) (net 5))
 (segment (start 179.99182 46.99) (end 178.7 48.28182) (width 0.1778) (layer B.Cu) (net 5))
 (segment (start 178.7 48.28182) (end 178.7 48.781802) (width 0.1778) (layer B.Cu) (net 5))
 (segment (start 180.34 43.18) (end 181.61 44.45) (width 0.1778) (layer B.Cu) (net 5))
 (segment (start 181.61 46.355) (end 180.975 46.99) (width 0.1778) (layer B.Cu) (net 5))
 (via (at 178.7 49.1) (size 0.45) (drill 0.3) (layers F.Cu B.Cu) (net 5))
 (segment (start 174.5622 48.46) (end 174.530484 48.491716) (width 0.1778) (layer F.Cu) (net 10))
 (segment (start 175.14 48.46) (end 174.5622 48.46) (width 0.1778) (layer F.Cu) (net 10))
 (segment (start 173.863982 48.491716) (end 173.608298 48.236032) (width 0.1778) (layer F.Cu) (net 10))
 (segment (start 173.608298 47.591702) (end 173.875001 47.324999) (width 0.1778) (layer F.Cu) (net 10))
 (segment (start 173.875001 47.324999) (end 174.1 47.1) (width 0.1778) (layer F.Cu) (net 10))
 (segment (start 173.608298 48.236032) (end 173.608298 47.591702) (width 0.1778) (layer F.Cu) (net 10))
 (segment (start 174.530484 48.491716) (end 173.863982 48.491716) (width 0.1778) (layer F.Cu) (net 10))
 (segment (start 167.64 48.26) (end 172.94 48.26) (width 0.1778) (layer B.Cu) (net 10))
 (segment (start 172.94 48.26) (end 173.875001 47.324999) (width 0.1778) (layer B.Cu) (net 10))
 (via (at 174.1 47.1) (size 0.45) (drill 0.3) (layers F.Cu B.Cu) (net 10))
 (segment (start 173.875001 47.324999) (end 174.1 47.1) (width 0.1778) (layer B.Cu) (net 10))
 (segment (start 180.34 45.72) (end 177.7 48.36) (width 0.1778) (layer B.Cu) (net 6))
 (segment (start 177.7 48.36) (end 177.7 48.6) (width 0.1778) (layer B.Cu) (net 6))
 (segment (start 177.475001 48.824999) (end 177.7 48.6) (width 0.1778) (layer F.Cu) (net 6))
 (segment (start 177.44 48.86) (end 177.475001 48.824999) (width 0.1778) (layer F.Cu) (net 6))
 (segment (start 175.14 48.86) (end 177.44 48.86) (width 0.1778) (layer F.Cu) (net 6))
 (via (at 177.7 48.6) (size 0.45) (drill 0.3) (layers F.Cu B.Cu) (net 6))
 (segment (start 175.14 47.66) (end 174.44 47.66) (width 0.1778) (layer F.Cu) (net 9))
 (segment (start 171.3 50.8) (end 173.875001 48.224999) (width 0.1778) (layer B.Cu) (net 9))
 (segment (start 174.44 47.66) (end 174.324999 47.775001) (width 0.1778) (layer F.Cu) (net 9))
 (segment (start 174.324999 47.775001) (end 174.1 48) (width 0.1778) (layer F.Cu) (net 9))
 (segment (start 173.875001 48.224999) (end 174.1 48) (width 0.1778) (layer B.Cu) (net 9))
 (segment (start 167.64 50.8) (end 171.3 50.8) (width 0.1778) (layer B.Cu) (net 9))
 (via (at 174.1 48) (size 0.45) (drill 0.3) (layers F.Cu B.Cu) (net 9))
 (segment (start 179.124 48.06) (end 179.324 48.26) (width 0.1778) (layer F.Cu) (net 7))
 (segment (start 175.14 48.06) (end 179.124 48.06) (width 0.1778) (layer F.Cu) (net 7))
 (segment (start 179.324 48.26) (end 180.34 48.26) (width 0.1778) (layer F.Cu) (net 7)))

